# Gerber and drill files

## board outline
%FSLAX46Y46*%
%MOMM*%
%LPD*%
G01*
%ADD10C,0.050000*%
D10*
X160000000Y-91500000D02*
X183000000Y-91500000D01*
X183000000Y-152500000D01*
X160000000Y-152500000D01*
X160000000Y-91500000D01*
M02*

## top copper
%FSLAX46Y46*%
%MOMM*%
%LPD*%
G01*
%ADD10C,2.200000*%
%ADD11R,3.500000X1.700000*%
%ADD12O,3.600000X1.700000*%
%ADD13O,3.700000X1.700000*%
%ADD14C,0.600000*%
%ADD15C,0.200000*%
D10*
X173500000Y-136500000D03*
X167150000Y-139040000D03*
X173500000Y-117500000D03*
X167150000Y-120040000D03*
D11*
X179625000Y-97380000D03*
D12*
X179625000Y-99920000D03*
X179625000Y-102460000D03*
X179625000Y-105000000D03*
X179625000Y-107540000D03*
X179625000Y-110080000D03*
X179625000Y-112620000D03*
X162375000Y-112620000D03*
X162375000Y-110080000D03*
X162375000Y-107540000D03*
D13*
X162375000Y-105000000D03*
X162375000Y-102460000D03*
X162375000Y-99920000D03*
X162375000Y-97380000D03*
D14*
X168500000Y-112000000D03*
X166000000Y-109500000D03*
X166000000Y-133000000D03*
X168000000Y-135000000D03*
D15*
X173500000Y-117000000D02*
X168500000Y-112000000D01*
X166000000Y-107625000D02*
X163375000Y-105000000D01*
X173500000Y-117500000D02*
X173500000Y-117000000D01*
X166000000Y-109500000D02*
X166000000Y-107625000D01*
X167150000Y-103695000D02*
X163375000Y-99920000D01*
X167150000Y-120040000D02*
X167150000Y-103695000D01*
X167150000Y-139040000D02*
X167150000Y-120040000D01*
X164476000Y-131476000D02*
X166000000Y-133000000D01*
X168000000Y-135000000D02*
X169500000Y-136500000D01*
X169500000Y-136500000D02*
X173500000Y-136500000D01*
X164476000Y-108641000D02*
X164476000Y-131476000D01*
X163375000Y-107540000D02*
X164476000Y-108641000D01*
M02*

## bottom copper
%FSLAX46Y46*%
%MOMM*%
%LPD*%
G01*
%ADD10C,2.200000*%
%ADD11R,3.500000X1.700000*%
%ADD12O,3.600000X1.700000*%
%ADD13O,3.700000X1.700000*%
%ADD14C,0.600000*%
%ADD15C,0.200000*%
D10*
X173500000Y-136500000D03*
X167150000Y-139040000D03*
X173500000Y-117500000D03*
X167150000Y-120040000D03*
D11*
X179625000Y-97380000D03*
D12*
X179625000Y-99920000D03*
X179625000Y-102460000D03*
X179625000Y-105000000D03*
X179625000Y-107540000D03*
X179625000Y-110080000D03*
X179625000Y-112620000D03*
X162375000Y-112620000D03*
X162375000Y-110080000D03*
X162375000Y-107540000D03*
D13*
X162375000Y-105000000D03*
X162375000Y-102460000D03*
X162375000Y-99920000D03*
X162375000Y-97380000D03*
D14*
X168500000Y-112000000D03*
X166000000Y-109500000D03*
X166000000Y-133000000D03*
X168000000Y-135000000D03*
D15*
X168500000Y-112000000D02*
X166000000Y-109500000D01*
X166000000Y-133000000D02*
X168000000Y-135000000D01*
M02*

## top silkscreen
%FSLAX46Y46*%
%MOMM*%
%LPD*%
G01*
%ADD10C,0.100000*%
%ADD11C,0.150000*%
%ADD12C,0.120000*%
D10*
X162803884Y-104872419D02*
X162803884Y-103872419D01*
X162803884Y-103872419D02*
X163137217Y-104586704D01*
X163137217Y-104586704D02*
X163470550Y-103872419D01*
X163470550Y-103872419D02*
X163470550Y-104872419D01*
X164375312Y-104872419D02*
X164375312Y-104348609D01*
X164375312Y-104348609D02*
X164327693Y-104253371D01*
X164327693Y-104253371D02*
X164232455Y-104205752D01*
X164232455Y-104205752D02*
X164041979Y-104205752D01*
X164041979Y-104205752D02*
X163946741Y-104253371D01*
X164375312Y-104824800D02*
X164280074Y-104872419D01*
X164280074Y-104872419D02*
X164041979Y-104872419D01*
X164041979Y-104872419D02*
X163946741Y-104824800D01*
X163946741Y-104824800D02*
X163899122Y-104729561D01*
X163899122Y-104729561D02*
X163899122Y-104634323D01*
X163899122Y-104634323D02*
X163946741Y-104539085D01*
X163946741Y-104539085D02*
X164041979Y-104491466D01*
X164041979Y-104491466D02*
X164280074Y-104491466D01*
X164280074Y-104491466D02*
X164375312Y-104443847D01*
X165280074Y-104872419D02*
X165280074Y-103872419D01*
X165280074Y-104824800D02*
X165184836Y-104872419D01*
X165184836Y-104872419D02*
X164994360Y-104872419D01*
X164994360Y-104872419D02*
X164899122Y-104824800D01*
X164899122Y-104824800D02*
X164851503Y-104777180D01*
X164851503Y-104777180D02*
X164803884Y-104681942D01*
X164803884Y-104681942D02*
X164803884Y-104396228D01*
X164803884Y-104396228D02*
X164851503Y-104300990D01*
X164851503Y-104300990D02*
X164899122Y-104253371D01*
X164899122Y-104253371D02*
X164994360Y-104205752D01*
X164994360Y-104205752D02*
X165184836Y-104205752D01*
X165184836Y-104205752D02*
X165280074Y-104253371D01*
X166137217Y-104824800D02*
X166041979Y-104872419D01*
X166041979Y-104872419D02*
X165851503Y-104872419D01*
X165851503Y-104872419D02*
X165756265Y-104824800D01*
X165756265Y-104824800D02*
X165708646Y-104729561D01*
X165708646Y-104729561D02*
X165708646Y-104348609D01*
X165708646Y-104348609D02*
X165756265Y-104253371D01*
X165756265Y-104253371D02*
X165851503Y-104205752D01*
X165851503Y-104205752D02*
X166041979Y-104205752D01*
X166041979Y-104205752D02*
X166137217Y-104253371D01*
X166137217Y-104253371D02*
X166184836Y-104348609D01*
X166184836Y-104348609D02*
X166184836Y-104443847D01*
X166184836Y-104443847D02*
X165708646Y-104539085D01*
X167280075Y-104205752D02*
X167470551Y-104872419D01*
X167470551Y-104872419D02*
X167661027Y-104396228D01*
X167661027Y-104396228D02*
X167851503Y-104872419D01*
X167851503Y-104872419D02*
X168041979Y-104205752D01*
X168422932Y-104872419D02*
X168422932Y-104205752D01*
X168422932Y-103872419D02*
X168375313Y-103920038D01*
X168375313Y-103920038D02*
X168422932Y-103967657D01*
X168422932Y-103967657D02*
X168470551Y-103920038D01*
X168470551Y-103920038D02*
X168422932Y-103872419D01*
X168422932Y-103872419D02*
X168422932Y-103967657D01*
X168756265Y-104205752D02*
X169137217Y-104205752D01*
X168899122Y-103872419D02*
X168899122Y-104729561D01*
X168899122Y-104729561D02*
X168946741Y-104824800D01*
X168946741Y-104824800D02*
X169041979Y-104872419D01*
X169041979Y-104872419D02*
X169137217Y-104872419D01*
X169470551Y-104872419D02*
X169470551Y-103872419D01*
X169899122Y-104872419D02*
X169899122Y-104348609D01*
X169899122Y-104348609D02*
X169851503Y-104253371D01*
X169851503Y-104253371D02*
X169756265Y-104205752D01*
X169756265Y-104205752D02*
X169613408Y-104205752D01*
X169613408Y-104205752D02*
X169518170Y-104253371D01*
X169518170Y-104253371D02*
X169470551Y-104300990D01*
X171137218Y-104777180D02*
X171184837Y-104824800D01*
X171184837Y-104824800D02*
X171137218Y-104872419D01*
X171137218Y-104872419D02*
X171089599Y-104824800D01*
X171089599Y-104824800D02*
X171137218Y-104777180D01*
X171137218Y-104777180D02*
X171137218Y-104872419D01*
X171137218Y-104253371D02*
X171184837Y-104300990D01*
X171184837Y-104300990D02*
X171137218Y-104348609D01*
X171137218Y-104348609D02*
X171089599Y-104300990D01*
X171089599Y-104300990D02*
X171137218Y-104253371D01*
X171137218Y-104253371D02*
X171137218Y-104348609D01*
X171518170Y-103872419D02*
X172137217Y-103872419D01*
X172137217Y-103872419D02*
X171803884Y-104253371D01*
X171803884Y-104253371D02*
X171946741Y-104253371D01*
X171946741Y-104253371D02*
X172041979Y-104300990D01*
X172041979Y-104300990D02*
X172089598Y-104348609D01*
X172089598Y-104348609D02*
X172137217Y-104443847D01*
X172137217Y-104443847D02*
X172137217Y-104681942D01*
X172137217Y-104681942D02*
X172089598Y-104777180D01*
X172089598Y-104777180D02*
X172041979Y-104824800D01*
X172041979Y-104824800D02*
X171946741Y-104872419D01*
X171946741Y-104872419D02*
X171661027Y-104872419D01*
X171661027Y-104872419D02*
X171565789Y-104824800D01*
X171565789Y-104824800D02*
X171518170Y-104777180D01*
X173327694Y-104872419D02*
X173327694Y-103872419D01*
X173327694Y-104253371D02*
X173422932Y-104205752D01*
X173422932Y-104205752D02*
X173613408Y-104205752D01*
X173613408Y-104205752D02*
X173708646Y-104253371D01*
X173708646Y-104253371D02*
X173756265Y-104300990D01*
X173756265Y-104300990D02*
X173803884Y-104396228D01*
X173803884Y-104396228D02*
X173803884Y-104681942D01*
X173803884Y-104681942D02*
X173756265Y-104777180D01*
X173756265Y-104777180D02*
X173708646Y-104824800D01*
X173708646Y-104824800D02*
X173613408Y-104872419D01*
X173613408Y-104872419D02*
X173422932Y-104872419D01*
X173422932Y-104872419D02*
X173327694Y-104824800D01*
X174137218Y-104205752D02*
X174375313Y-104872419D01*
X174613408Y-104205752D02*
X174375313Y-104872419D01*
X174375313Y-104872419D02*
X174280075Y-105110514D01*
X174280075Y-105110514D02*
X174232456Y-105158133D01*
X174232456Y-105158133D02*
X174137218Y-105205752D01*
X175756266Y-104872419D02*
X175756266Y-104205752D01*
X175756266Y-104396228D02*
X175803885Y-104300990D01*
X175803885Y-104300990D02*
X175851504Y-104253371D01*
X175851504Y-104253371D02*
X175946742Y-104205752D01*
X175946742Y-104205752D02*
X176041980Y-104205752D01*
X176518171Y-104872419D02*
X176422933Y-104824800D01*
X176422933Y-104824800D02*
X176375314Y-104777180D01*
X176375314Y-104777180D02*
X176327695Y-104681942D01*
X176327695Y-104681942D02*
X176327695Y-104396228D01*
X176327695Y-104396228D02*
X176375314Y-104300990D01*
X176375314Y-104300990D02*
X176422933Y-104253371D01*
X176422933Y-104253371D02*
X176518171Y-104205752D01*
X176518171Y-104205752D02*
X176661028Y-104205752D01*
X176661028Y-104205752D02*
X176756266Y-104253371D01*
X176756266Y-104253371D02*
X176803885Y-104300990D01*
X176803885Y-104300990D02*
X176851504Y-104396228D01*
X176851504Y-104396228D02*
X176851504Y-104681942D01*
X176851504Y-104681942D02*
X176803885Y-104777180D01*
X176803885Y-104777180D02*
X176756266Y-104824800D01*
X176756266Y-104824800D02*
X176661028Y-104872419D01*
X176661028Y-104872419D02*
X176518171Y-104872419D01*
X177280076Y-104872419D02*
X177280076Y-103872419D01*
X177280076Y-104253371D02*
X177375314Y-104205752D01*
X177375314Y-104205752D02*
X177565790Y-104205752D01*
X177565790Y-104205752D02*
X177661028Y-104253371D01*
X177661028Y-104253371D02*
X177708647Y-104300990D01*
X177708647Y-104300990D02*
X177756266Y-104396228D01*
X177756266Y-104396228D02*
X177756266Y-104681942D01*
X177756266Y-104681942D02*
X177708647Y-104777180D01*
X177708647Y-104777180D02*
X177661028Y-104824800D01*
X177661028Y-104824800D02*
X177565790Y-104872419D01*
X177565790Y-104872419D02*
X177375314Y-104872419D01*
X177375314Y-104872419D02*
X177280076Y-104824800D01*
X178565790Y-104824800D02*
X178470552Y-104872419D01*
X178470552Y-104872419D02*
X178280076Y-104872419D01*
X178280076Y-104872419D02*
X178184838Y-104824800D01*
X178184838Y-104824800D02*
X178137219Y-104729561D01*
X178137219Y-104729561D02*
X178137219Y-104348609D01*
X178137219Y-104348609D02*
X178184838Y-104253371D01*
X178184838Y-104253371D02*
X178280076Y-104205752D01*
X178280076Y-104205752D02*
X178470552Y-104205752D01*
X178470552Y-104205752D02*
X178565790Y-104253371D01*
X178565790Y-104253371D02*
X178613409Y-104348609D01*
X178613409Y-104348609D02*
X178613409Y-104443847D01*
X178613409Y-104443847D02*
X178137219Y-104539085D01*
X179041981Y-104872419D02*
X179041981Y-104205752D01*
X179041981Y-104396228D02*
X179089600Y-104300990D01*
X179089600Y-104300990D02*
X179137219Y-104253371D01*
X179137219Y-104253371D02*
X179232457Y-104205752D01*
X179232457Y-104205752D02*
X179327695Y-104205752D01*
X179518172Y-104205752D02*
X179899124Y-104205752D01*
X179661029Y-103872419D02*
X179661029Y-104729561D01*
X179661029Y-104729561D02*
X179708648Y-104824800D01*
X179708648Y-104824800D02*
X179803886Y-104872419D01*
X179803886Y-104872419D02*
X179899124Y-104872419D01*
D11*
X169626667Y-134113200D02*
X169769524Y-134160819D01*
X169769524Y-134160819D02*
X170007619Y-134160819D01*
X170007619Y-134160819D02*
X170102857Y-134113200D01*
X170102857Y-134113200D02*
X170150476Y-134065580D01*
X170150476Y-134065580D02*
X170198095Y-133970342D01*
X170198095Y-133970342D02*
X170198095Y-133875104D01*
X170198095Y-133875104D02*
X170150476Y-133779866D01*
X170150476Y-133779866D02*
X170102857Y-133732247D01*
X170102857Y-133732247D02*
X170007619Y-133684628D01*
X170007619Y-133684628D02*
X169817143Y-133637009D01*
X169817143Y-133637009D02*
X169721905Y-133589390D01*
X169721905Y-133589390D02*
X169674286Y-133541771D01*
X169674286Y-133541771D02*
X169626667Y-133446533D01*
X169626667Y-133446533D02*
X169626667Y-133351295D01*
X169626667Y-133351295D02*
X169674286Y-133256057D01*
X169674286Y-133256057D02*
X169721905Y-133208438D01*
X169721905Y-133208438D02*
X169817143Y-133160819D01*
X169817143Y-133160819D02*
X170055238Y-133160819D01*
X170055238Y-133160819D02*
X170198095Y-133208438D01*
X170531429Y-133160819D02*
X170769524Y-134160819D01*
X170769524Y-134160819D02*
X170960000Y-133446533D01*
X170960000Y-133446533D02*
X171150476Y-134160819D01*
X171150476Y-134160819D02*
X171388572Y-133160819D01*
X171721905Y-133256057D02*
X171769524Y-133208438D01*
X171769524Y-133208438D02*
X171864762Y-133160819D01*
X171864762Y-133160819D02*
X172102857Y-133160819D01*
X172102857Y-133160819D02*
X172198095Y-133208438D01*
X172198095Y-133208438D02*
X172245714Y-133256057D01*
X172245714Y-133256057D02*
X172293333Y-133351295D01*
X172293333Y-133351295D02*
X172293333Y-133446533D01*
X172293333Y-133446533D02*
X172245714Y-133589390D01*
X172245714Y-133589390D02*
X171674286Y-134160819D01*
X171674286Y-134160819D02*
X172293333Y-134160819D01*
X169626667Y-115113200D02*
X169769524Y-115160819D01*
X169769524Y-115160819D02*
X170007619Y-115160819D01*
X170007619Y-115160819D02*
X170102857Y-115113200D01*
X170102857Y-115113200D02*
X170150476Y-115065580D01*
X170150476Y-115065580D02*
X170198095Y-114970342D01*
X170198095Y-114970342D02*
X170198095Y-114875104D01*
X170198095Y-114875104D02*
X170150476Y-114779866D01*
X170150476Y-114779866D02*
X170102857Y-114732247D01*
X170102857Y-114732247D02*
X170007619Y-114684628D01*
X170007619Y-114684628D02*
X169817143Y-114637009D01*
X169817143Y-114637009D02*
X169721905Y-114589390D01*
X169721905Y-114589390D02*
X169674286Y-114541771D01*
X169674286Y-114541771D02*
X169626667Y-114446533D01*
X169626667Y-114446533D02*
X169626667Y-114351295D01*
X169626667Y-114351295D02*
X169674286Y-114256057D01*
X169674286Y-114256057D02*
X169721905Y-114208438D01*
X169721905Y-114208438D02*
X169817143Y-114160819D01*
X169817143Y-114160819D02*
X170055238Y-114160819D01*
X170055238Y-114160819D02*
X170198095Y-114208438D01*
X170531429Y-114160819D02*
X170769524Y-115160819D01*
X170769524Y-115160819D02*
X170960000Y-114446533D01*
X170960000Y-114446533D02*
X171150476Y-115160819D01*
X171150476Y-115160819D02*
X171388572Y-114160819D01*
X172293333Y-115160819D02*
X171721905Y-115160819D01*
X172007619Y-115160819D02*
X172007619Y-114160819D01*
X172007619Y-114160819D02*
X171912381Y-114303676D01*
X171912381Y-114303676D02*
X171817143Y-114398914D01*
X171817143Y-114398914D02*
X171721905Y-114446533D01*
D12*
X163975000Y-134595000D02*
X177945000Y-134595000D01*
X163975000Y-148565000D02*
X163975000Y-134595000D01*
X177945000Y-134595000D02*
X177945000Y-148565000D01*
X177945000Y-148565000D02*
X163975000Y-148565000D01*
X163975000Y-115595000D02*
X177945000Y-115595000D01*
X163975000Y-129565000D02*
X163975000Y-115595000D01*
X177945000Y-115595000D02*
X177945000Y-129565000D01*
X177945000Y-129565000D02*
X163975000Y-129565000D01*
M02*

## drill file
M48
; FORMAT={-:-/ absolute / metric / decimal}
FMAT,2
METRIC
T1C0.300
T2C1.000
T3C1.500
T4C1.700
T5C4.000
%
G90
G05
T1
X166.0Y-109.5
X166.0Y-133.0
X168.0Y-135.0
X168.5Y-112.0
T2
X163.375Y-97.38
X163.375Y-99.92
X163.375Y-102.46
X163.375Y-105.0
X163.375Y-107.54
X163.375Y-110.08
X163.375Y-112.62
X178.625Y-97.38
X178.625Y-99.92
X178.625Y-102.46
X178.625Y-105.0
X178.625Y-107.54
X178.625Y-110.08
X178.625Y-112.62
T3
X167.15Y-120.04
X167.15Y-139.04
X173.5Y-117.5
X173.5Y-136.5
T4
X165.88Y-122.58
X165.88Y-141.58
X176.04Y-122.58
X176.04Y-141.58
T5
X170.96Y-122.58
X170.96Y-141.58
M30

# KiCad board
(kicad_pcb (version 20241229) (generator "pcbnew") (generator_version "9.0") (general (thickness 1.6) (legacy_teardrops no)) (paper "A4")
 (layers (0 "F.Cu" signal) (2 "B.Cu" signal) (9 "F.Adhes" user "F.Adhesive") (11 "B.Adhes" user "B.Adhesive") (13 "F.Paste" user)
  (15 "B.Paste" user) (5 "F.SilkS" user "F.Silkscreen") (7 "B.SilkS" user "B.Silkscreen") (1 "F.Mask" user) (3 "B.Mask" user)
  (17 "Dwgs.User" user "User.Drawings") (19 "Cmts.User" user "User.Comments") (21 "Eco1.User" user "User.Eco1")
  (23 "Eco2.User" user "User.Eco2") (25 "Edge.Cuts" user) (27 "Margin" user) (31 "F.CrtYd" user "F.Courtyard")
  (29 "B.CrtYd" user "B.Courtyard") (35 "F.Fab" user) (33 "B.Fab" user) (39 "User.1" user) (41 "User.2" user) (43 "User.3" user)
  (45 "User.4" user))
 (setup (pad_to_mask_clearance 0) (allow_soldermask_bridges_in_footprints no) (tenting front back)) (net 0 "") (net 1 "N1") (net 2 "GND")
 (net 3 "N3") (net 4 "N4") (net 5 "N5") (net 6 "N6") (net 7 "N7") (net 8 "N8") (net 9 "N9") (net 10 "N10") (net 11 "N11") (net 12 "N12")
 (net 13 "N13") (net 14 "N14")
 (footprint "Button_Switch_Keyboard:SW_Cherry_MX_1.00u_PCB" (layer "F.Cu") (at 173.5 136.5)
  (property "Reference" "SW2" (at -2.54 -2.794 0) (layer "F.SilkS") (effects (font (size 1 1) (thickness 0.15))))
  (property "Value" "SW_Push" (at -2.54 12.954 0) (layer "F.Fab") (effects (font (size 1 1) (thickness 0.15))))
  (fp_line (start -9.525 -1.905) (end 4.445 -1.905) (stroke (width 0.12) (type solid)) (layer "F.SilkS"))
  (fp_line (start -9.525 12.065) (end -9.525 -1.905) (stroke (width 0.12) (type solid)) (layer "F.SilkS"))
  (fp_line (start 4.445 -1.905) (end 4.445 12.065) (stroke (width 0.12) (type solid)) (layer "F.SilkS"))
  (fp_line (start 4.445 12.065) (end -9.525 12.065) (stroke (width 0.12) (type solid)) (layer "F.SilkS"))
  (pad "" np_thru_hole circle (at -7.62 5.08) (size 1.7 1.7) (drill 1.7) (layers "*.Cu" "*.Mask"))
  (pad "" np_thru_hole circle (at -2.54 5.08) (size 4 4) (drill 4) (layers "*.Cu" "*.Mask"))
  (pad "" np_thru_hole circle (at 2.54 5.08) (size 1.7 1.7) (drill 1.7) (layers "*.Cu" "*.Mask"))
  (pad "1" thru_hole circle (at 0 0) (size 2.2 2.2) (drill 1.5) (layers "*.Cu" "*.Mask") (remove_unused_layers no) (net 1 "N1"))
  (pad "2" thru_hole circle (at -6.35 2.54) (size 2.2 2.2) (drill 1.5) (layers "*.Cu" "*.Mask") (remove_unused_layers no) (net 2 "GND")))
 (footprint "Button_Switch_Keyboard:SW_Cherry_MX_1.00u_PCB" (layer "F.Cu") (at 173.5 117.5)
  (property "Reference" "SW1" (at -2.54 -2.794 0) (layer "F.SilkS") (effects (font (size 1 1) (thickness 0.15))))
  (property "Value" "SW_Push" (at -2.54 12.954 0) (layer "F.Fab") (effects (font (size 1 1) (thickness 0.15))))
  (fp_line (start -9.525 -1.905) (end 4.445 -1.905) (stroke (width 0.12) (type solid)) (layer "F.SilkS"))
  (fp_line (start -9.525 12.065) (end -9.525 -1.905) (stroke (width 0.12) (type solid)) (layer "F.SilkS"))
  (fp_line (start 4.445 -1.905) (end 4.445 12.065) (stroke (width 0.12) (type solid)) (layer "F.SilkS"))
  (fp_line (start 4.445 12.065) (end -9.525 12.065) (stroke (width 0.12) (type solid)) (layer "F.SilkS"))
  (pad "" np_thru_hole circle (at -7.62 5.08) (size 1.7 1.7) (drill 1.7) (layers "*.Cu" "*.Mask"))
  (pad "" np_thru_hole circle (at -2.54 5.08) (size 4 4) (drill 4) (layers "*.Cu" "*.Mask"))
  (pad "" np_thru_hole circle (at 2.54 5.08) (size 1.7 1.7) (drill 1.7) (layers "*.Cu" "*.Mask"))
  (pad "1" thru_hole circle (at 0 0) (size 2.2 2.2) (drill 1.5) (layers "*.Cu" "*.Mask") (remove_unused_layers no) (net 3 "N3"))
  (pad "2" thru_hole circle (at -6.35 2.54) (size 2.2 2.2) (drill 1.5) (layers "*.Cu" "*.Mask") (remove_unused_layers no) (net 2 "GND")))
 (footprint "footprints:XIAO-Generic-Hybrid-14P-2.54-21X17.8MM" (layer "B.Cu") (at 171 105 180)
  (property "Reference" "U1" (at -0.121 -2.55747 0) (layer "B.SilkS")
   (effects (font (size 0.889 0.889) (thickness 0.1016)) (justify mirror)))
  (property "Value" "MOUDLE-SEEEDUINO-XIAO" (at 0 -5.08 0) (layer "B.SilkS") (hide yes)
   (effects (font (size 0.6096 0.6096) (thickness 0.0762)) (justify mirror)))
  (pad "1" thru_hole rect (at -7.625 7.62 180) (size 3.5 1.7) (drill 1 (offset -1 0)) (layers "*.Cu" "*.Mask") (remove_unused_layers no)
   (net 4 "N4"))
  (pad "2" thru_hole oval (at -7.625 5.08 180) (size 3.6 1.7) (drill 1 (offset -1 0)) (layers "*.Cu" "*.Mask") (remove_unused_layers no)
   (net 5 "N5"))
  (pad "3" thru_hole oval (at -7.625 2.54 180) (size 3.6 1.7) (drill 1 (offset -1 0)) (layers "*.Cu" "*.Mask") (remove_unused_layers no)
   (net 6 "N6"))
  (pad "4" thru_hole oval (at -7.625 0 180) (size 3.6 1.7) (drill 1 (offset -1 0)) (layers "*.Cu" "*.Mask") (remove_unused_layers no)
   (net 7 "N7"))
  (pad "5" thru_hole oval (at -7.625 -2.54 180) (size 3.6 1.7) (drill 1 (offset -1 0)) (layers "*.Cu" "*.Mask") (remove_unused_layers no)
   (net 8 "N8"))
  (pad "6" thru_hole oval (at -7.625 -5.08) (size 3.6 1.7) (drill 1 (offset 1 0)) (layers "*.Cu" "*.Mask") (remove_unused_layers no)
   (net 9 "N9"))
  (pad "7" thru_hole oval (at -7.625 -7.62 180) (size 3.6 1.7) (drill 1 (offset -1 0)) (layers "*.Cu" "*.Mask") (remove_unused_layers no)
   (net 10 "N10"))
  (pad "8" thru_hole oval (at 7.625 -7.62 180) (size 3.6 1.7) (drill 1 (offset 1 0)) (layers "*.Cu" "*.Mask") (remove_unused_layers no)
   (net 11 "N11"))
  (pad "9" thru_hole oval (at 7.625 -5.08 180) (size 3.6 1.7) (drill 1 (offset 1 0)) (layers "*.Cu" "*.Mask") (remove_unused_layers no)
   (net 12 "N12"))
  (pad "10" thru_hole oval (at 7.625 -2.54 180) (size 3.6 1.7) (drill 1 (offset 1 0)) (layers "*.Cu" "*.Mask") (remove_unused_layers no)
   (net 1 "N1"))
  (pad "11" thru_hole oval (at 7.625 0 180) (size 3.7 1.7) (drill 1 (offset 1 0)) (layers "*.Cu" "*.Mask") (remove_unused_layers no)
   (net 3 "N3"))
  (pad "12" thru_hole oval (at 7.625 2.54 180) (size 3.7 1.7) (drill 1 (offset 1 0)) (layers "*.Cu" "*.Mask") (remove_unused_layers no)
   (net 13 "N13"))
  (pad "13" thru_hole oval (at 7.625 5.08 180) (size 3.7 1.7) (drill 1 (offset 1 0)) (layers "*.Cu" "*.Mask") (remove_unused_layers no)
   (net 2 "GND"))
  (pad "14" thru_hole oval (at 7.625 7.62 180) (size 3.7 1.7) (drill 1 (offset 1 0)) (layers "*.Cu" "*.Mask") (remove_unused_layers no)
   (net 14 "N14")))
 (gr_rect (start 160 91.5) (end 183 152.5) (stroke (width 0.05) (type default)) (fill no) (layer "Edge.Cuts"))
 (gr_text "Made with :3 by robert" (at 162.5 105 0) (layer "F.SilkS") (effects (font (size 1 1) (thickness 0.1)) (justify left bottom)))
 (segment (start 173.5 117) (end 168.5 112) (width 0.2) (layer "F.Cu") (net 3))
 (segment (start 166 107.625) (end 163.375 105) (width 0.2) (layer "F.Cu") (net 3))
 (segment (start 173.5 117.5) (end 173.5 117) (width 0.2) (layer "F.Cu") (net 3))
 (segment (start 166 109.5) (end 166 107.625) (width 0.2) (layer "F.Cu") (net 3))
 (via (at 168.5 112) (size 0.6) (drill 0.3) (layers "F.Cu" "B.Cu") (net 3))
 (via (at 166 109.5) (size 0.6) (drill 0.3) (layers "F.Cu" "B.Cu") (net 3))
 (segment (start 168.5 112) (end 166 109.5) (width 0.2) (layer "B.Cu") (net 3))
 (segment (start 167.15 103.695) (end 163.375 99.92) (width 0.2) (layer "F.Cu") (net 2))
 (segment (start 167.15 120.04) (end 167.15 103.695) (width 0.2) (layer "F.Cu") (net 2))
 (segment (start 167.15 139.04) (end 167.15 120.04) (width 0.2) (layer "F.Cu") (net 2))
 (segment (start 164.476 131.476) (end 166 133) (width 0.2) (layer "F.Cu") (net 1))
 (segment (start 168 135) (end 169.5 136.5) (width 0.2) (layer "F.Cu") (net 1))
 (segment (start 169.5 136.5) (end 173.5 136.5) (width 0.2) (layer "F.Cu") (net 1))
 (segment (start 164.476 108.641) (end 164.476 131.476) (width 0.2) (layer "F.Cu") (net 1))
 (segment (start 163.375 107.54) (end 164.476 108.641) (width 0.2) (layer "F.Cu") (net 1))
 (via (at 166 133) (size 0.6) (drill 0.3) (layers "F.Cu" "B.Cu") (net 1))
 (via (at 168 135) (size 0.6) (drill 0.3) (layers "F.Cu" "B.Cu") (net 1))
 (segment (start 166 133) (end 168 135) (width 0.2) (layer "B.Cu") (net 1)))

